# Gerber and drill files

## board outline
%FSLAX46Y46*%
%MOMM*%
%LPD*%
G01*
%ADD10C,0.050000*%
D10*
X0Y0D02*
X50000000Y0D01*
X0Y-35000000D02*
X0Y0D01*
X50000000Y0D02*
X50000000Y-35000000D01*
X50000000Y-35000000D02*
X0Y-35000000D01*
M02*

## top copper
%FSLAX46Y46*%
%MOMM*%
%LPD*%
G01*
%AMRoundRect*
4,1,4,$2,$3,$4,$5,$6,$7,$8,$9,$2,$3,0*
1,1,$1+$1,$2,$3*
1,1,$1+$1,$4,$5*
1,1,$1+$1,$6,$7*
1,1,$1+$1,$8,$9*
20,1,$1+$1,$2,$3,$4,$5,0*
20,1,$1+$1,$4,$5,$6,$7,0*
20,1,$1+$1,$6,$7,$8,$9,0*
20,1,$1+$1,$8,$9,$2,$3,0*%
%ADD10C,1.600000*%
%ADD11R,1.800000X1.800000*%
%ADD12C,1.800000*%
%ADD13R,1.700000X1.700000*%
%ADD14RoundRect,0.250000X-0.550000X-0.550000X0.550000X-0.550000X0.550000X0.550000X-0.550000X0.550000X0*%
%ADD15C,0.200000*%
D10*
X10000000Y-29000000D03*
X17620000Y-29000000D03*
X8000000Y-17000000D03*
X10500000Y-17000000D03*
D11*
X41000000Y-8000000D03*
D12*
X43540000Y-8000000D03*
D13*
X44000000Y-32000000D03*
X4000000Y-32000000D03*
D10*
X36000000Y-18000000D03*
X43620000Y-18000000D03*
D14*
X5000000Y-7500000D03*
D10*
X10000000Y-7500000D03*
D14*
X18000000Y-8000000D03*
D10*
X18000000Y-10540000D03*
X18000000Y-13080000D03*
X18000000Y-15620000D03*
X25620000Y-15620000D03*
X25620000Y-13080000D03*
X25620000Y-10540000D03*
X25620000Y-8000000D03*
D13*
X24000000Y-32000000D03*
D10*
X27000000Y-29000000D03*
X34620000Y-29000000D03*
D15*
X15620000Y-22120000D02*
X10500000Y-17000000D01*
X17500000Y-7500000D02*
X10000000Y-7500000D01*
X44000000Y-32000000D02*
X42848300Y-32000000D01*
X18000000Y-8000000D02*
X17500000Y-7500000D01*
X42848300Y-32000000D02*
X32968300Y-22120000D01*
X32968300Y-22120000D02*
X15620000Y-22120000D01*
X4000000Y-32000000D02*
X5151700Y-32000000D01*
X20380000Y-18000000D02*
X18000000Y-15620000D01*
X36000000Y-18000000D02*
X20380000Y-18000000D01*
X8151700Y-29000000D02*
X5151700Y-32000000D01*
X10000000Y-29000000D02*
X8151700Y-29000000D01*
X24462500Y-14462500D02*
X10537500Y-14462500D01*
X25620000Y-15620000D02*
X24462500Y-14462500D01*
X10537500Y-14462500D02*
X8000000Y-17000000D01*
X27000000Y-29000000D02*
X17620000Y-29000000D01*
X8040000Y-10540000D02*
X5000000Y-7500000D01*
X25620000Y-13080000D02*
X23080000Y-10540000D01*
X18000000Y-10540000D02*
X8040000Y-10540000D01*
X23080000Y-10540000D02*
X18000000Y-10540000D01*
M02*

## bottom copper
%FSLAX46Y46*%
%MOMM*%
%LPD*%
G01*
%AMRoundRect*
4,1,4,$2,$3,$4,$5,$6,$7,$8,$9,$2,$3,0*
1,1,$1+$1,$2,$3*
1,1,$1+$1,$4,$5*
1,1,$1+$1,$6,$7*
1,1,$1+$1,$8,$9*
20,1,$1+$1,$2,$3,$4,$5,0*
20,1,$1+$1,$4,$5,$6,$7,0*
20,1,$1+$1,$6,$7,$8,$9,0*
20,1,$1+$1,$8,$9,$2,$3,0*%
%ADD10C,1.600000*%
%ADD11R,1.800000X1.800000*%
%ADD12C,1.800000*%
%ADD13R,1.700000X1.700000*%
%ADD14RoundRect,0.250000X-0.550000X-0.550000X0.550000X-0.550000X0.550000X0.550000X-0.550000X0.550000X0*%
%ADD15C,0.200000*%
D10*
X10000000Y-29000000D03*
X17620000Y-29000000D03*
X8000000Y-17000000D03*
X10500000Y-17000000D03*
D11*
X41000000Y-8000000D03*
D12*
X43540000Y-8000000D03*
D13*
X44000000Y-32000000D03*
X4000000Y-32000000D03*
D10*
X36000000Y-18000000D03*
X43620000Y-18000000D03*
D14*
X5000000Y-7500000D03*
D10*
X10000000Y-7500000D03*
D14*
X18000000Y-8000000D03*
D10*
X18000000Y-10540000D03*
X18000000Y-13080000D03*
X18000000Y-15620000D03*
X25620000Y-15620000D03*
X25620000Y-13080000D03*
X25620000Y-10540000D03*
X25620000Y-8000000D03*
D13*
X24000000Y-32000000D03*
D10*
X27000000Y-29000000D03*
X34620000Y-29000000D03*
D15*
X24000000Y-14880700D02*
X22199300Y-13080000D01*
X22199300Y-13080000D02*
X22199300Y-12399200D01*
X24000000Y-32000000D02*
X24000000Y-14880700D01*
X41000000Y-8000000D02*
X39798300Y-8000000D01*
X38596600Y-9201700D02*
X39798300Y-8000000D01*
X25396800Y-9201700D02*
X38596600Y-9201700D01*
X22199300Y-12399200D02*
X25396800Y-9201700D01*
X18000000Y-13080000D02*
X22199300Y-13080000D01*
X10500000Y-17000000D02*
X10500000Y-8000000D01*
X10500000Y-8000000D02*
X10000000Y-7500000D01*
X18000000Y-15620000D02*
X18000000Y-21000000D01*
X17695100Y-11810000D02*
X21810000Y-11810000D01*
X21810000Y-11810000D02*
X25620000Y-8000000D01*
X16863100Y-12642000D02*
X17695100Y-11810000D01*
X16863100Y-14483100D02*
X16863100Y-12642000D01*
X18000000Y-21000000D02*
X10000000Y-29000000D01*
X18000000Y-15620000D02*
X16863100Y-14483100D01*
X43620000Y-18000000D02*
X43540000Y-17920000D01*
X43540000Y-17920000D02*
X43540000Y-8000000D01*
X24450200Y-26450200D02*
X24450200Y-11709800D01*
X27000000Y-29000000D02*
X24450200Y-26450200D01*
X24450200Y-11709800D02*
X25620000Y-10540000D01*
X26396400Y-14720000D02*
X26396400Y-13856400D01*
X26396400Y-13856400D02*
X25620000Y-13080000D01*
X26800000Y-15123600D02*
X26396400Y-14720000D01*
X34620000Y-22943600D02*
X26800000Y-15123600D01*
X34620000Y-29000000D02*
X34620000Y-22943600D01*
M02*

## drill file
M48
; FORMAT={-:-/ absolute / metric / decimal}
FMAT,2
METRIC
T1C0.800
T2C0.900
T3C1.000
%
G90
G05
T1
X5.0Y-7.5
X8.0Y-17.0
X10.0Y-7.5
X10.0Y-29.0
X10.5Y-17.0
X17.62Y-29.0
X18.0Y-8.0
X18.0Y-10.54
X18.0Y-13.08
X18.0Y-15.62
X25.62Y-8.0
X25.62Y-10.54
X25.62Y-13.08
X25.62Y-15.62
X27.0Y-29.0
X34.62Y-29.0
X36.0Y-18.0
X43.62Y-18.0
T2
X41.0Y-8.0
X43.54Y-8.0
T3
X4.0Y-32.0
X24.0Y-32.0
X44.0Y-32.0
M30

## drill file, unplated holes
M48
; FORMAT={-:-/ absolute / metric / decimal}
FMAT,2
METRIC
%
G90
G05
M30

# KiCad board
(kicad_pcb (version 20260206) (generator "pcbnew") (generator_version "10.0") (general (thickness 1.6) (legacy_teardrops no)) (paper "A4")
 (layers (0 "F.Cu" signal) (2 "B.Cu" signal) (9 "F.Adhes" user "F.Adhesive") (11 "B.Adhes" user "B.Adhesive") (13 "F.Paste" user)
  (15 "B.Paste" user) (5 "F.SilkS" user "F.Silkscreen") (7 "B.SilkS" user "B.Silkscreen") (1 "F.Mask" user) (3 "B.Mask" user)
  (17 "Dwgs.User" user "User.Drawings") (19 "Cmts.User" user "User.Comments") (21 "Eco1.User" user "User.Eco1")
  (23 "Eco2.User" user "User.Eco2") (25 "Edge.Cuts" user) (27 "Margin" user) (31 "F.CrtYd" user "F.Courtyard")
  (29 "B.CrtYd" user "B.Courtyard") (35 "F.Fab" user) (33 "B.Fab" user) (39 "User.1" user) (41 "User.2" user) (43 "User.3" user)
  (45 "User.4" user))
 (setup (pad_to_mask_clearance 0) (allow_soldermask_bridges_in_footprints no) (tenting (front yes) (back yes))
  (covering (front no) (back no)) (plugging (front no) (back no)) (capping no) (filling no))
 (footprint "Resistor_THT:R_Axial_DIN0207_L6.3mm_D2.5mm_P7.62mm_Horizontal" (layer "F.Cu") (at 10 29)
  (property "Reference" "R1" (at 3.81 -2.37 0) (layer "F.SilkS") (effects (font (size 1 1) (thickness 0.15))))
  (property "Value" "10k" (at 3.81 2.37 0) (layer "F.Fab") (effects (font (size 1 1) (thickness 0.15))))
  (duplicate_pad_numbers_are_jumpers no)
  (pad "1" thru_hole circle (at 0 0) (size 1.6 1.6) (drill 0.8) (layers "*.Cu" "*.Mask") (remove_unused_layers no) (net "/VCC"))
  (pad "2" thru_hole circle (at 7.62 0) (size 1.6 1.6) (drill 0.8) (layers "*.Cu" "*.Mask") (remove_unused_layers no) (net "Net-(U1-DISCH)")))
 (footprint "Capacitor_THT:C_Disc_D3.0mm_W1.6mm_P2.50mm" (layer "F.Cu") (at 8 17)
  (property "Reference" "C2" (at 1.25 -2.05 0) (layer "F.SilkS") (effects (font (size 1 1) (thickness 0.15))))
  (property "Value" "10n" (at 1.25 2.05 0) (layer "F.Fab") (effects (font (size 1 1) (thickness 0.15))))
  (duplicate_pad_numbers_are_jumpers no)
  (pad "1" thru_hole circle (at 0 0) (size 1.6 1.6) (drill 0.8) (layers "*.Cu" "*.Mask") (remove_unused_layers no) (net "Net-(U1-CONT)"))
  (pad "2" thru_hole circle (at 2.5 0) (size 1.6 1.6) (drill 0.8) (layers "*.Cu" "*.Mask") (remove_unused_layers no) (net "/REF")))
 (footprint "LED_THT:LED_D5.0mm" (layer "F.Cu") (at 41 8)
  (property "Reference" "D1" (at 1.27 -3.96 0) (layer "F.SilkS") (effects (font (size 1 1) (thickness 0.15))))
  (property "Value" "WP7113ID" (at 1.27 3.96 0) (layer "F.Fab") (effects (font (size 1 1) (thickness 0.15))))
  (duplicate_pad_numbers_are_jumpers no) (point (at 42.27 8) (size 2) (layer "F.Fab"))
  (pad "1" thru_hole rect (at 0 0) (size 1.8 1.8) (drill 0.9) (layers "*.Cu" "*.Mask") (remove_unused_layers no) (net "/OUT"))
  (pad "2" thru_hole circle (at 2.54 0) (size 1.8 1.8) (drill 0.9) (layers "*.Cu" "*.Mask") (remove_unused_layers no) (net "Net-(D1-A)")))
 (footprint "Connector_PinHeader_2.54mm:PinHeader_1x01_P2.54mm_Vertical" (layer "F.Cu") (at 44 32)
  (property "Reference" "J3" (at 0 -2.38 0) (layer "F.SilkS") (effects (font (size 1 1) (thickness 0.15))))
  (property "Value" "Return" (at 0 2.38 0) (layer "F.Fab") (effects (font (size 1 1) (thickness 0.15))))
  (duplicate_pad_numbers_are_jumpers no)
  (pad "1" thru_hole rect (at 0 0) (size 1.7 1.7) (drill 1) (layers "*.Cu" "*.Mask") (remove_unused_layers no) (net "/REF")))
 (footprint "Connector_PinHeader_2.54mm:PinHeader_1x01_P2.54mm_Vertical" (layer "F.Cu") (at 4 32)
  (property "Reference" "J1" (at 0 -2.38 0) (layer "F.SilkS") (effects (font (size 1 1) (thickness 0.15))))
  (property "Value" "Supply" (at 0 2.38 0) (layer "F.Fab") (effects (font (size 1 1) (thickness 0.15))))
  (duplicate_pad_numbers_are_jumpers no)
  (pad "1" thru_hole rect (at 0 0) (size 1.7 1.7) (drill 1) (layers "*.Cu" "*.Mask") (remove_unused_layers no) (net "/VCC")))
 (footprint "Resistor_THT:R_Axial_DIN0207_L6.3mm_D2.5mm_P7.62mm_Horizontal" (layer "F.Cu") (at 36 18)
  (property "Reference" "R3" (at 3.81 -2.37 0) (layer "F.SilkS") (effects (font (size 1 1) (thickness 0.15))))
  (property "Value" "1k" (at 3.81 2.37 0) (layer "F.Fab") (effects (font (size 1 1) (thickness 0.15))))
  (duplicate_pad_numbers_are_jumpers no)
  (pad "1" thru_hole circle (at 0 0) (size 1.6 1.6) (drill 0.8) (layers "*.Cu" "*.Mask") (remove_unused_layers no) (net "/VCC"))
  (pad "2" thru_hole circle (at 7.62 0) (size 1.6 1.6) (drill 0.8) (layers "*.Cu" "*.Mask") (remove_unused_layers no) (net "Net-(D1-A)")))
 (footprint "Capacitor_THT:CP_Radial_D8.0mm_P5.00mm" (layer "F.Cu") (at 5 7.5)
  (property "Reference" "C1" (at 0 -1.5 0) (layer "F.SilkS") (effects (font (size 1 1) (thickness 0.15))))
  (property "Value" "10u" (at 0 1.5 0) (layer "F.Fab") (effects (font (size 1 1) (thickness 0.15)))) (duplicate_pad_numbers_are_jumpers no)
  (pad "1" thru_hole roundrect (at 0 0) (size 1.6 1.6) (drill 0.8) (layers "*.Cu" "*.Mask") (remove_unused_layers no)
   (roundrect_rratio 0.15625) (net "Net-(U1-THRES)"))
  (pad "2" thru_hole circle (at 5 0) (size 1.6 1.6) (drill 0.8) (layers "*.Cu" "*.Mask") (remove_unused_layers no) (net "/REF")))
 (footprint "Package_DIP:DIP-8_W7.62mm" (layer "F.Cu") (at 18 8)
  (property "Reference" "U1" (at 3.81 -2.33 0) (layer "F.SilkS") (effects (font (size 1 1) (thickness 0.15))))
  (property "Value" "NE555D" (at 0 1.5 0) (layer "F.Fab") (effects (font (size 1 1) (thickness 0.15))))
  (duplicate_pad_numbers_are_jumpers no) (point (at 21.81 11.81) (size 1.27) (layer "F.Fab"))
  (pad "1" thru_hole roundrect (at 0 0) (size 1.6 1.6) (drill 0.8) (layers "*.Cu" "*.Mask") (remove_unused_layers no)
   (roundrect_rratio 0.15625) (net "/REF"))
  (pad "2" thru_hole circle (at 0 2.54) (size 1.6 1.6) (drill 0.8) (layers "*.Cu" "*.Mask") (remove_unused_layers no) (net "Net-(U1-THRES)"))
  (pad "3" thru_hole circle (at 0 5.08) (size 1.6 1.6) (drill 0.8) (layers "*.Cu" "*.Mask") (remove_unused_layers no) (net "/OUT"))
  (pad "4" thru_hole circle (at 0 7.62) (size 1.6 1.6) (drill 0.8) (layers "*.Cu" "*.Mask") (remove_unused_layers no) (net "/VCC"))
  (pad "5" thru_hole circle (at 7.62 7.62) (size 1.6 1.6) (drill 0.8) (layers "*.Cu" "*.Mask") (remove_unused_layers no)
   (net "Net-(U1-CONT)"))
  (pad "6" thru_hole circle (at 7.62 5.08) (size 1.6 1.6) (drill 0.8) (layers "*.Cu" "*.Mask") (remove_unused_layers no)
   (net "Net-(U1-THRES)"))
  (pad "7" thru_hole circle (at 7.62 2.54) (size 1.6 1.6) (drill 0.8) (layers "*.Cu" "*.Mask") (remove_unused_layers no)
   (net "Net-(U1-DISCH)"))
  (pad "8" thru_hole circle (at 7.62 0) (size 1.6 1.6) (drill 0.8) (layers "*.Cu" "*.Mask") (remove_unused_layers no) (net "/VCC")))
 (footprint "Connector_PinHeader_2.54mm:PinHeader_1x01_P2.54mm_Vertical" (layer "F.Cu") (at 24 32)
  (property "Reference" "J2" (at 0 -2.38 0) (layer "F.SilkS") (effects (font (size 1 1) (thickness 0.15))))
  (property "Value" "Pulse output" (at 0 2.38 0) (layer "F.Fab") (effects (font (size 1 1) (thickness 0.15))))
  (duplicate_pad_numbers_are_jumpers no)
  (pad "1" thru_hole rect (at 0 0) (size 1.7 1.7) (drill 1) (layers "*.Cu" "*.Mask") (remove_unused_layers no) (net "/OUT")))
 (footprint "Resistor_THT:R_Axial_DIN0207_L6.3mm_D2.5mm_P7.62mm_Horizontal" (layer "F.Cu") (at 27 29)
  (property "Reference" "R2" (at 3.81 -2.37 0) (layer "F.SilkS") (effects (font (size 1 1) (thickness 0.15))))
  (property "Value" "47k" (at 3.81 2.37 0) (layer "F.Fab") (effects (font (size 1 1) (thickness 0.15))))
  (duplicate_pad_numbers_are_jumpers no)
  (pad "1" thru_hole circle (at 0 0) (size 1.6 1.6) (drill 0.8) (layers "*.Cu" "*.Mask") (remove_unused_layers no) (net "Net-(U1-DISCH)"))
  (pad "2" thru_hole circle (at 7.62 0) (size 1.6 1.6) (drill 0.8) (layers "*.Cu" "*.Mask") (remove_unused_layers no) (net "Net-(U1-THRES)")))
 (gr_line (start 0 0) (end 50 0) (stroke (width 0.05) (type default)) (layer "Edge.Cuts"))
 (gr_line (start 0 35) (end 0 0) (stroke (width 0.05) (type default)) (layer "Edge.Cuts"))
 (gr_line (start 50 0) (end 50 35) (stroke (width 0.05) (type default)) (layer "Edge.Cuts"))
 (gr_line (start 50 35) (end 0 35) (stroke (width 0.05) (type default)) (layer "Edge.Cuts"))
 (segment (start 24 14.8807) (end 22.1993 13.08) (width 0.2) (layer "B.Cu") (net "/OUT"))
 (segment (start 22.1993 13.08) (end 22.1993 12.3992) (width 0.2) (layer "B.Cu") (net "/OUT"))
 (segment (start 24 32) (end 24 14.8807) (width 0.2) (layer "B.Cu") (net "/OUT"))
 (segment (start 41 8) (end 39.7983 8) (width 0.2) (layer "B.Cu") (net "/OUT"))
 (segment (start 38.5966 9.2017) (end 39.7983 8) (width 0.2) (layer "B.Cu") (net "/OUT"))
 (segment (start 25.3968 9.2017) (end 38.5966 9.2017) (width 0.2) (layer "B.Cu") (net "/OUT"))
 (segment (start 22.1993 12.3992) (end 25.3968 9.2017) (width 0.2) (layer "B.Cu") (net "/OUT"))
 (segment (start 18 13.08) (end 22.1993 13.08) (width 0.2) (layer "B.Cu") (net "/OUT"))
 (segment (start 15.62 22.12) (end 10.5 17) (width 0.2) (layer "F.Cu") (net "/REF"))
 (segment (start 17.5 7.5) (end 10 7.5) (width 0.2) (layer "F.Cu") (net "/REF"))
 (segment (start 44 32) (end 42.8483 32) (width 0.2) (layer "F.Cu") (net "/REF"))
 (segment (start 18 8) (end 17.5 7.5) (width 0.2) (layer "F.Cu") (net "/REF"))
 (segment (start 42.8483 32) (end 32.9683 22.12) (width 0.2) (layer "F.Cu") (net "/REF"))
 (segment (start 32.9683 22.12) (end 15.62 22.12) (width 0.2) (layer "F.Cu") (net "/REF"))
 (segment (start 10.5 17) (end 10.5 8) (width 0.2) (layer "B.Cu") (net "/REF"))
 (segment (start 10.5 8) (end 10 7.5) (width 0.2) (layer "B.Cu") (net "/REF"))
 (segment (start 4 32) (end 5.1517 32) (width 0.2) (layer "F.Cu") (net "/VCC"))
 (segment (start 20.38 18) (end 18 15.62) (width 0.2) (layer "F.Cu") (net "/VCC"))
 (segment (start 36 18) (end 20.38 18) (width 0.2) (layer "F.Cu") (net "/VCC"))
 (segment (start 8.1517 29) (end 5.1517 32) (width 0.2) (layer "F.Cu") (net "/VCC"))
 (segment (start 10 29) (end 8.1517 29) (width 0.2) (layer "F.Cu") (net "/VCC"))
 (segment (start 18 15.62) (end 18 21) (width 0.2) (layer "B.Cu") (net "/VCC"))
 (segment (start 17.6951 11.81) (end 21.81 11.81) (width 0.2) (layer "B.Cu") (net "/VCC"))
 (segment (start 21.81 11.81) (end 25.62 8) (width 0.2) (layer "B.Cu") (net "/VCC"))
 (segment (start 16.8631 12.642) (end 17.6951 11.81) (width 0.2) (layer "B.Cu") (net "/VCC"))
 (segment (start 16.8631 14.4831) (end 16.8631 12.642) (width 0.2) (layer "B.Cu") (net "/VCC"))
 (segment (start 18 21) (end 10 29) (width 0.2) (layer "B.Cu") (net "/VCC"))
 (segment (start 18 15.62) (end 16.8631 14.4831) (width 0.2) (layer "B.Cu") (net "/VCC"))
 (segment (start 43.62 18) (end 43.54 17.92) (width 0.2) (layer "B.Cu") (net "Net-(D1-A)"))
 (segment (start 43.54 17.92) (end 43.54 8) (width 0.2) (layer "B.Cu") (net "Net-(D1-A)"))
 (segment (start 24.4625 14.4625) (end 10.5375 14.4625) (width 0.2) (layer "F.Cu") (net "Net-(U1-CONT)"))
 (segment (start 25.62 15.62) (end 24.4625 14.4625) (width 0.2) (layer "F.Cu") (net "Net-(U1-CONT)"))
 (segment (start 10.5375 14.4625) (end 8 17) (width 0.2) (layer "F.Cu") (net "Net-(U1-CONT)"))
 (segment (start 27 29) (end 17.62 29) (width 0.2) (layer "F.Cu") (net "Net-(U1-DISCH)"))
 (segment (start 24.4502 26.4502) (end 24.4502 11.7098) (width 0.2) (layer "B.Cu") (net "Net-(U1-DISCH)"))
 (segment (start 27 29) (end 24.4502 26.4502) (width 0.2) (layer "B.Cu") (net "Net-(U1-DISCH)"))
 (segment (start 24.4502 11.7098) (end 25.62 10.54) (width 0.2) (layer "B.Cu") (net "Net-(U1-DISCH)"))
 (segment (start 8.04 10.54) (end 5 7.5) (width 0.2) (layer "F.Cu") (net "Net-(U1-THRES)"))
 (segment (start 25.62 13.08) (end 23.08 10.54) (width 0.2) (layer "F.Cu") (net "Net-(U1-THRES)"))
 (segment (start 18 10.54) (end 8.04 10.54) (width 0.2) (layer "F.Cu") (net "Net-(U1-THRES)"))
 (segment (start 23.08 10.54) (end 18 10.54) (width 0.2) (layer "F.Cu") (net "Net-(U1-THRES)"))
 (segment (start 26.3964 14.72) (end 26.3964 13.8564) (width 0.2) (layer "B.Cu") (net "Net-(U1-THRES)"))
 (segment (start 26.3964 13.8564) (end 25.62 13.08) (width 0.2) (layer "B.Cu") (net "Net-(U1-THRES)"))
 (segment (start 26.8 15.1236) (end 26.3964 14.72) (width 0.2) (layer "B.Cu") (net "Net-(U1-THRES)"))
 (segment (start 34.62 22.9436) (end 26.8 15.1236) (width 0.2) (layer "B.Cu") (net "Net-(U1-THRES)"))
 (segment (start 34.62 29) (end 34.62 22.9436) (width 0.2) (layer "B.Cu") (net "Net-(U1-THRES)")))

